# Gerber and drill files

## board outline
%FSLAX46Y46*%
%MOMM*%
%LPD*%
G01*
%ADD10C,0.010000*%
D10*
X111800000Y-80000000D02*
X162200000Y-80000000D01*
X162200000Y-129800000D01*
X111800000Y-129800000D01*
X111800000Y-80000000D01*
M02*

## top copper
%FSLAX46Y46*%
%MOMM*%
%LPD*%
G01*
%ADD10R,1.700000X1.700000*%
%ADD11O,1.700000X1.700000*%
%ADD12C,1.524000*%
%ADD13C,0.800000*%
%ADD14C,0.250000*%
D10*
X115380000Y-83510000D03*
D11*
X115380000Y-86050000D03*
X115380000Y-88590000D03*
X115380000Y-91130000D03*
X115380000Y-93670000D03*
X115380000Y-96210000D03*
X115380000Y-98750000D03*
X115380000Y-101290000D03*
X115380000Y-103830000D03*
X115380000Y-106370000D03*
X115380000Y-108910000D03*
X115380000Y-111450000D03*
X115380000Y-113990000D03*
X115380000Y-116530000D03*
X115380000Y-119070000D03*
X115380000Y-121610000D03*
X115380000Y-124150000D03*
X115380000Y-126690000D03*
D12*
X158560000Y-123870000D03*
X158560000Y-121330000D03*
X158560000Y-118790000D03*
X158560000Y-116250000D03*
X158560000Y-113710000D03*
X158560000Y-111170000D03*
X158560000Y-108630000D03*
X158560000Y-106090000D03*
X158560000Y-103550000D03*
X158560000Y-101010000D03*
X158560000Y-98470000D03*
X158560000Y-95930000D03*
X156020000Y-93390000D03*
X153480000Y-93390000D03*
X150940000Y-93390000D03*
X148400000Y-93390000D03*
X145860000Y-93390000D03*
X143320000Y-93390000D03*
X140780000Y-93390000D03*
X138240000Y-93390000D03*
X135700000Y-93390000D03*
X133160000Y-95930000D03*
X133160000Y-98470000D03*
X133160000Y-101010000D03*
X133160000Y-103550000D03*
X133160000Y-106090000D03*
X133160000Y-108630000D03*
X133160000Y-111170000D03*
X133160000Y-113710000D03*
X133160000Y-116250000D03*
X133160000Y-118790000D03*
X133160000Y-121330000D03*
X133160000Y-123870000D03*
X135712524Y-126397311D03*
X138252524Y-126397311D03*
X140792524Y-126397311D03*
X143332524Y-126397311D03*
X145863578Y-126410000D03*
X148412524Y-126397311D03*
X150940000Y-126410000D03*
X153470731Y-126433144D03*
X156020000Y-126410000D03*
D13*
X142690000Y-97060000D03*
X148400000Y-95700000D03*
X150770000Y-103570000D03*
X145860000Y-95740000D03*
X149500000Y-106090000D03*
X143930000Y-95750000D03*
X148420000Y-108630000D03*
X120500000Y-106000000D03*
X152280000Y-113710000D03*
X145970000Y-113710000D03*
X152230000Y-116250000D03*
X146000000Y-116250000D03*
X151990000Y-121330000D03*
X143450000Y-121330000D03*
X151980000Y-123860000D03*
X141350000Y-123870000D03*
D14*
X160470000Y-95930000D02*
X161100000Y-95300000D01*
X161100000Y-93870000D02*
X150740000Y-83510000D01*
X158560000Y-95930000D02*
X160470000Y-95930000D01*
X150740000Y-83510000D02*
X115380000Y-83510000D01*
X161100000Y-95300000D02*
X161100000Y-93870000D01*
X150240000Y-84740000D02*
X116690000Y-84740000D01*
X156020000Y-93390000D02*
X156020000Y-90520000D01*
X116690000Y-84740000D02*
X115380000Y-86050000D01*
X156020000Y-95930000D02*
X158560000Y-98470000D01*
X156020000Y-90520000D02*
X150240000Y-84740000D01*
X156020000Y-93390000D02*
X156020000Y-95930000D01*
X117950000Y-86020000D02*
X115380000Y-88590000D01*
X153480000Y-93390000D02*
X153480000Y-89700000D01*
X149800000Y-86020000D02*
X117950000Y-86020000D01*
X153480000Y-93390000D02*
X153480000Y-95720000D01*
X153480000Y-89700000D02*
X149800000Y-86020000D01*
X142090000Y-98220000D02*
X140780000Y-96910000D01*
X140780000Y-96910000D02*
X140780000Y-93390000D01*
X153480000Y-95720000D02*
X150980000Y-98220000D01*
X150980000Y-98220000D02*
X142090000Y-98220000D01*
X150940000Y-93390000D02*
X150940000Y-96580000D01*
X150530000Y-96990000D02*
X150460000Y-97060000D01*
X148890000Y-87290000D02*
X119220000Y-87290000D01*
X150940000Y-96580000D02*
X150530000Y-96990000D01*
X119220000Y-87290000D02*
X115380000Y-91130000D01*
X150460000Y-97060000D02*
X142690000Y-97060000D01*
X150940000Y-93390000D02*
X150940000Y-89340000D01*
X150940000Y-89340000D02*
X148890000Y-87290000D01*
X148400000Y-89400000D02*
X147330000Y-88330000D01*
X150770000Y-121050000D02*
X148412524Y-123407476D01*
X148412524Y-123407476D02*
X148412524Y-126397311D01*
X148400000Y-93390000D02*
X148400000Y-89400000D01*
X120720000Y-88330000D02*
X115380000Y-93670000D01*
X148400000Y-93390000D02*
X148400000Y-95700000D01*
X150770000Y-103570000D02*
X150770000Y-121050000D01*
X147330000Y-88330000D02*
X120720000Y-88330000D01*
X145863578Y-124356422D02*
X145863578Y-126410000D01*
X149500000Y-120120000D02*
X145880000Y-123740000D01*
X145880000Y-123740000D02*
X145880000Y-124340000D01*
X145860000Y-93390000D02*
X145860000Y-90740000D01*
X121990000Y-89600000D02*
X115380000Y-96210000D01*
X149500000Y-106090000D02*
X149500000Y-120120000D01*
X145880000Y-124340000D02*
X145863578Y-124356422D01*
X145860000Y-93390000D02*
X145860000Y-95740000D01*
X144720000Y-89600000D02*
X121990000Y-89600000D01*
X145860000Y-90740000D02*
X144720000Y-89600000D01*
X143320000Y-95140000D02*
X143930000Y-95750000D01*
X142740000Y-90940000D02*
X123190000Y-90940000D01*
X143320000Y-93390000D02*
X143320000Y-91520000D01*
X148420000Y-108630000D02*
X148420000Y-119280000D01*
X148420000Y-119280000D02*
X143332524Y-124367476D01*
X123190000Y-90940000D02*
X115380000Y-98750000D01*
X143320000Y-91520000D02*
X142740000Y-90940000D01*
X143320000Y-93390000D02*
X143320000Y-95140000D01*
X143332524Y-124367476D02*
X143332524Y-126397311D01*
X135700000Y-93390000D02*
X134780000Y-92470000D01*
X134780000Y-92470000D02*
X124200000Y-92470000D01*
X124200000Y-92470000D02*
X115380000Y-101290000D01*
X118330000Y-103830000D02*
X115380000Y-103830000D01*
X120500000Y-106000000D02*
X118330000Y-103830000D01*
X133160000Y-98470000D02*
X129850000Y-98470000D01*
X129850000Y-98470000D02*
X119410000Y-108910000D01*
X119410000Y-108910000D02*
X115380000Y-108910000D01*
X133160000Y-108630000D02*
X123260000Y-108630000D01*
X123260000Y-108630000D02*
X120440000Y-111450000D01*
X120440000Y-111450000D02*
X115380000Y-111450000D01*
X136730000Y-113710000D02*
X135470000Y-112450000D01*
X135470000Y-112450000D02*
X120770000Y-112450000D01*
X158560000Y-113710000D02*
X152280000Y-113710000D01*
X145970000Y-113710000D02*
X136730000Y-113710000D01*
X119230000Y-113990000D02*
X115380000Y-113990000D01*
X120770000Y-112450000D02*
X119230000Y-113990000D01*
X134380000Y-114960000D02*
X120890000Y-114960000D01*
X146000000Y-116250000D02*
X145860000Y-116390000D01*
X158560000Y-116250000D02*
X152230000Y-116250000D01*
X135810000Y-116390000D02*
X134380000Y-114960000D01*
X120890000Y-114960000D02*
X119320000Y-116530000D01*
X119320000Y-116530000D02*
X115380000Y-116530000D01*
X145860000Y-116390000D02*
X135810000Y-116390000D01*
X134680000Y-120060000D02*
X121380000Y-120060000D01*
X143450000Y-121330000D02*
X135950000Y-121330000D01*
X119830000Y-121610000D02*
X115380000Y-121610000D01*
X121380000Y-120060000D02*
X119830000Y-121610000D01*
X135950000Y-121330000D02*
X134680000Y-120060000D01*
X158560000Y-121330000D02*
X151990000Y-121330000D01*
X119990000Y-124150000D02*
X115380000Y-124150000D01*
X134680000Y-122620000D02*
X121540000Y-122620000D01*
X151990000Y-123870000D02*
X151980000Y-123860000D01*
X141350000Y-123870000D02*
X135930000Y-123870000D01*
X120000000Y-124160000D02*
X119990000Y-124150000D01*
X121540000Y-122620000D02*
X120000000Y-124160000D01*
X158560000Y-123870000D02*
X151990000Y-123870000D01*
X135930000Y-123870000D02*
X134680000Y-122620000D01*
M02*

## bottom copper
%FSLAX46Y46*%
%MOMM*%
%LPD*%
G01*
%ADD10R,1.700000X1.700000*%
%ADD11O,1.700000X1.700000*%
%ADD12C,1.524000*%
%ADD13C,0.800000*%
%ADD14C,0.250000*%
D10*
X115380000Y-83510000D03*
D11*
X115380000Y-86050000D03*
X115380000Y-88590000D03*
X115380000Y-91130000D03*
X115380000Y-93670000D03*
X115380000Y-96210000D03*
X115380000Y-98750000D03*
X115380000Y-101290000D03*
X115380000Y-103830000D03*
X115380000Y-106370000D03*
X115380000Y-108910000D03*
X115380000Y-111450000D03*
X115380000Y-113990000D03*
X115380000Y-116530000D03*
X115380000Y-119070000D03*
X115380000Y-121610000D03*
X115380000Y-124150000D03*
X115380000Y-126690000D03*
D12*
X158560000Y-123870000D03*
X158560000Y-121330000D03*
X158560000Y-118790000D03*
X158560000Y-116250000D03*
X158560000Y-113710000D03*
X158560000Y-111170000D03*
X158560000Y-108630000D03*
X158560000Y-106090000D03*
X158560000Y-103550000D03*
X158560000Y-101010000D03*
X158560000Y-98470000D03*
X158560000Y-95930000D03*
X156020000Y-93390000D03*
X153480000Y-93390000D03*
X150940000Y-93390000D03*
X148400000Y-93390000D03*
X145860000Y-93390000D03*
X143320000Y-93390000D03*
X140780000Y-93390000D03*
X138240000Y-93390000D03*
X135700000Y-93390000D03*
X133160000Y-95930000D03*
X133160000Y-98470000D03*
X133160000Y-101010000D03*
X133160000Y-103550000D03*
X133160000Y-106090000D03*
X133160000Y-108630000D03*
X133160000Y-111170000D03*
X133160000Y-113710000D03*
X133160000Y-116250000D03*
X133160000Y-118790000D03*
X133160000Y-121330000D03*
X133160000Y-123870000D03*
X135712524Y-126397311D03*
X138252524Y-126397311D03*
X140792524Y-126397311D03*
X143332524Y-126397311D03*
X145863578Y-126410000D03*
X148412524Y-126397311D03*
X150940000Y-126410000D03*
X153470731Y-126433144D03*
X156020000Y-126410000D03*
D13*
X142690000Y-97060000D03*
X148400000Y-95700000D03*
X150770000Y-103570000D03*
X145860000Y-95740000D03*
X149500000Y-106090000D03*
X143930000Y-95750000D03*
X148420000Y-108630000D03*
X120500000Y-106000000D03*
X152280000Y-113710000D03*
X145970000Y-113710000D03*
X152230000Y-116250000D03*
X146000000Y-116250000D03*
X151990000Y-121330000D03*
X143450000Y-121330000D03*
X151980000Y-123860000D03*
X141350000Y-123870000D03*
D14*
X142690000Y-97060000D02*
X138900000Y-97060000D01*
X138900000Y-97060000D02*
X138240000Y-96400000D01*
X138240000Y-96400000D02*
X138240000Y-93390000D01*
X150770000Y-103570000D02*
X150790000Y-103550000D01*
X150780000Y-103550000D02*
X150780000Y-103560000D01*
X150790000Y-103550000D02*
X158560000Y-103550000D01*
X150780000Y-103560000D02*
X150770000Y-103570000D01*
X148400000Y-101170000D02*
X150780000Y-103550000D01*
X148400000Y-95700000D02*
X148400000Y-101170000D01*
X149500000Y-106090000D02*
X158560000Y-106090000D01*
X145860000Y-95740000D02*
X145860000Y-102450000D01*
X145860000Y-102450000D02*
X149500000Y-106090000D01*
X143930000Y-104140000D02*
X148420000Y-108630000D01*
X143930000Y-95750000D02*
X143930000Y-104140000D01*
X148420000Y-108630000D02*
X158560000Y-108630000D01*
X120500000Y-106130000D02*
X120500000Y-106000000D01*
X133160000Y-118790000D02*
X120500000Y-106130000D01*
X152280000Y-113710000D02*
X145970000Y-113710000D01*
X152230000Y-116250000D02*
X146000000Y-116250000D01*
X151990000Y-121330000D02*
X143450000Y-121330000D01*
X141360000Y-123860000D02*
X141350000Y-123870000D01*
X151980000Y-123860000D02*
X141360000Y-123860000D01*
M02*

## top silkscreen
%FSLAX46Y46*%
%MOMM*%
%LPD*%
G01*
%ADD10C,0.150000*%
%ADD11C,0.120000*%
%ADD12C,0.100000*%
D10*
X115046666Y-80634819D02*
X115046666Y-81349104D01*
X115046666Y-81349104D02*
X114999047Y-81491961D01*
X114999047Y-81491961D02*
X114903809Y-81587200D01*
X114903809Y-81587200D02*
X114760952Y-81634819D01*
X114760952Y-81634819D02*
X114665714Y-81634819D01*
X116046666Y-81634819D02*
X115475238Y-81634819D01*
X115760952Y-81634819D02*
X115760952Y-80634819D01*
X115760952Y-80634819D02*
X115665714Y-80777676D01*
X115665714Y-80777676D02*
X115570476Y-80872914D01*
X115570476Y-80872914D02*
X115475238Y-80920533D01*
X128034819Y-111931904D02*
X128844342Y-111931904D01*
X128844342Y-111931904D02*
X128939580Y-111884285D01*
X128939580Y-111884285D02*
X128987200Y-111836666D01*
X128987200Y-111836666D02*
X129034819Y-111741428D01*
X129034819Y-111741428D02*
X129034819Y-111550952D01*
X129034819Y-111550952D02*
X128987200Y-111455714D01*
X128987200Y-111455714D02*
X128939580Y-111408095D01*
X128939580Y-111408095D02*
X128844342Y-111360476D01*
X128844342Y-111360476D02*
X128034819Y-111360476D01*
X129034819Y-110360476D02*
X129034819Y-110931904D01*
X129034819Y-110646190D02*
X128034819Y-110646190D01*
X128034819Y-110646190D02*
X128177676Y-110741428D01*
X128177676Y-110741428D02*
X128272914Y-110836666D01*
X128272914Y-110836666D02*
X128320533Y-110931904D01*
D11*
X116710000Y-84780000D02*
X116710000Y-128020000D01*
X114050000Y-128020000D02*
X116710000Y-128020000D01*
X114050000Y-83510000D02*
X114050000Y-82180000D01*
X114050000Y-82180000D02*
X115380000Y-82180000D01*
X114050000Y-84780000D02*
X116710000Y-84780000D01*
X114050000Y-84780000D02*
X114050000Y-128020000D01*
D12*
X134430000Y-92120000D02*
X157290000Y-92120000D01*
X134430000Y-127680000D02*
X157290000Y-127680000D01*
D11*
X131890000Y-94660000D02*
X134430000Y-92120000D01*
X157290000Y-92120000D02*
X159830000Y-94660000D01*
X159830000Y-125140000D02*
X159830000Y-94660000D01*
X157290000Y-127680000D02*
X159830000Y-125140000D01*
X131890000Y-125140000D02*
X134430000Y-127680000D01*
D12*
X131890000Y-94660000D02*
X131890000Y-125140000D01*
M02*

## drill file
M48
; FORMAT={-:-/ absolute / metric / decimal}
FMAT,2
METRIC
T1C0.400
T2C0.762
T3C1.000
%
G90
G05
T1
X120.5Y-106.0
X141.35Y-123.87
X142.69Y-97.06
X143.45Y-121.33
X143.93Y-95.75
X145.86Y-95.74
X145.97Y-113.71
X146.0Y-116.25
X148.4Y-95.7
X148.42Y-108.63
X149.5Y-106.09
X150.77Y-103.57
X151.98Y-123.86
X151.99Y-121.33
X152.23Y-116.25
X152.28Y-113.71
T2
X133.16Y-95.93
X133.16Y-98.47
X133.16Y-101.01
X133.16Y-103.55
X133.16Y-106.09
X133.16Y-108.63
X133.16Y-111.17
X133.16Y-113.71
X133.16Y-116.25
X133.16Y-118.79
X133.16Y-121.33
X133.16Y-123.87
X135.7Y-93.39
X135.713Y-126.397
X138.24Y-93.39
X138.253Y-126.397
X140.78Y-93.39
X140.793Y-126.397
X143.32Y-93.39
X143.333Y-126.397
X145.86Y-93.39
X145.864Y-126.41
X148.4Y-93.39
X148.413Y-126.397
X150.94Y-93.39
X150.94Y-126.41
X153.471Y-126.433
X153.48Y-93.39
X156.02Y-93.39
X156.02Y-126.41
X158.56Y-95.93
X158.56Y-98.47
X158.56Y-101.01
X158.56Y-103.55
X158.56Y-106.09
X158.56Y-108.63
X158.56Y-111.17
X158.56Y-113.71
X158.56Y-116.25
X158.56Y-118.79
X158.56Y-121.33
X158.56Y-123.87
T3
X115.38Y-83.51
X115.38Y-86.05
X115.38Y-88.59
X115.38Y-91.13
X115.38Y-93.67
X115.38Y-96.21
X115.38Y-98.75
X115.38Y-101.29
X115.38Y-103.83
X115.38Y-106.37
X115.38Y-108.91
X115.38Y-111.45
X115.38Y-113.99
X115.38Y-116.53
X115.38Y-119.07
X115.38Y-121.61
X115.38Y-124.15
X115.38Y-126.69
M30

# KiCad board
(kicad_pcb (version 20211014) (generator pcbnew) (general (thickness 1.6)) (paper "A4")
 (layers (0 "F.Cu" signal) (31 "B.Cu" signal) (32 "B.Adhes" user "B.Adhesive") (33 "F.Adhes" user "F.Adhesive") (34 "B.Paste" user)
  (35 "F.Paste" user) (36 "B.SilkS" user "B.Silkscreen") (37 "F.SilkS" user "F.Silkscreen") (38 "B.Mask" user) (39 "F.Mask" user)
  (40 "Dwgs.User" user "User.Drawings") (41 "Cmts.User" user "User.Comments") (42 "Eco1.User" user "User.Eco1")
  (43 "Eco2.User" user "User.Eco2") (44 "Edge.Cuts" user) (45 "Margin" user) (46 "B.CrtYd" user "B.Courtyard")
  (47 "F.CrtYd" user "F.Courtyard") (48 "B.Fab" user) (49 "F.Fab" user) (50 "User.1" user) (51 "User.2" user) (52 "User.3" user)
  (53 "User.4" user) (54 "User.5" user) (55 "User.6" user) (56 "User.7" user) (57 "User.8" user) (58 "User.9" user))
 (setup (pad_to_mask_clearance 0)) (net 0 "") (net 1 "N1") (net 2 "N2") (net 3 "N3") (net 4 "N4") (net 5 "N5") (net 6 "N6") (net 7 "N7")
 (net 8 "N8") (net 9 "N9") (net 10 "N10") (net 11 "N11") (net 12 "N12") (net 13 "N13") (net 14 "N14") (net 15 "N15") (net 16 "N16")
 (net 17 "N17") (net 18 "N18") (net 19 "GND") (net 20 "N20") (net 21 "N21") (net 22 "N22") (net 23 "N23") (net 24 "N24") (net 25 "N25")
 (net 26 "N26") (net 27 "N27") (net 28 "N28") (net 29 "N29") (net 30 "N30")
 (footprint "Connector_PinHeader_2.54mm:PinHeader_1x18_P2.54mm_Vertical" (layer "F.Cu") (at 115.38 83.51)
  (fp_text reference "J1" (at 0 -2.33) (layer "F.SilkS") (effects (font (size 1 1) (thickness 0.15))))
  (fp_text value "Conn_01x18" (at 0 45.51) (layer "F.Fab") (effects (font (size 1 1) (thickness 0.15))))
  (fp_line (start 1.33 1.27) (end 1.33 44.51) (layer "F.SilkS") (width 0.12))
  (fp_line (start -1.33 44.51) (end 1.33 44.51) (layer "F.SilkS") (width 0.12))
  (fp_line (start -1.33 0) (end -1.33 -1.33) (layer "F.SilkS") (width 0.12))
  (fp_line (start -1.33 -1.33) (end 0 -1.33) (layer "F.SilkS") (width 0.12))
  (fp_line (start -1.33 1.27) (end 1.33 1.27) (layer "F.SilkS") (width 0.12))
  (fp_line (start -1.33 1.27) (end -1.33 44.51) (layer "F.SilkS") (width 0.12))
  (pad "1" thru_hole rect locked (at 0 0) (size 1.7 1.7) (drill 1) (layers *.Cu *.Mask) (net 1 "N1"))
  (pad "2" thru_hole oval locked (at 0 2.54) (size 1.7 1.7) (drill 1) (layers *.Cu *.Mask) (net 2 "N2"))
  (pad "3" thru_hole oval locked (at 0 5.08) (size 1.7 1.7) (drill 1) (layers *.Cu *.Mask) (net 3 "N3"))
  (pad "4" thru_hole oval locked (at 0 7.62) (size 1.7 1.7) (drill 1) (layers *.Cu *.Mask) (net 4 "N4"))
  (pad "5" thru_hole oval locked (at 0 10.16) (size 1.7 1.7) (drill 1) (layers *.Cu *.Mask) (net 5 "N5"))
  (pad "6" thru_hole oval locked (at 0 12.7) (size 1.7 1.7) (drill 1) (layers *.Cu *.Mask) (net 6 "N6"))
  (pad "7" thru_hole oval locked (at 0 15.24) (size 1.7 1.7) (drill 1) (layers *.Cu *.Mask) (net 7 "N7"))
  (pad "8" thru_hole oval locked (at 0 17.78) (size 1.7 1.7) (drill 1) (layers *.Cu *.Mask) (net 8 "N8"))
  (pad "9" thru_hole oval locked (at 0 20.32) (size 1.7 1.7) (drill 1) (layers *.Cu *.Mask) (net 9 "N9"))
  (pad "10" thru_hole oval locked (at 0 22.86) (size 1.7 1.7) (drill 1) (layers *.Cu *.Mask) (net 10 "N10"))
  (pad "11" thru_hole oval locked (at 0 25.4) (size 1.7 1.7) (drill 1) (layers *.Cu *.Mask) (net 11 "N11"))
  (pad "12" thru_hole oval locked (at 0 27.94) (size 1.7 1.7) (drill 1) (layers *.Cu *.Mask) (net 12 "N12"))
  (pad "13" thru_hole oval locked (at 0 30.48) (size 1.7 1.7) (drill 1) (layers *.Cu *.Mask) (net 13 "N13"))
  (pad "14" thru_hole oval locked (at 0 33.02) (size 1.7 1.7) (drill 1) (layers *.Cu *.Mask) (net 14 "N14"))
  (pad "15" thru_hole oval locked (at 0 35.56) (size 1.7 1.7) (drill 1) (layers *.Cu *.Mask) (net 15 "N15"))
  (pad "16" thru_hole oval locked (at 0 38.1) (size 1.7 1.7) (drill 1) (layers *.Cu *.Mask) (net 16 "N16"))
  (pad "17" thru_hole oval locked (at 0 40.64) (size 1.7 1.7) (drill 1) (layers *.Cu *.Mask) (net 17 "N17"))
  (pad "18" thru_hole oval locked (at 0 43.18) (size 1.7 1.7) (drill 1) (layers *.Cu *.Mask) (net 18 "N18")))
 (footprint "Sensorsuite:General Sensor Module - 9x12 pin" (layer "F.Cu") (at 145.86 111.17 90)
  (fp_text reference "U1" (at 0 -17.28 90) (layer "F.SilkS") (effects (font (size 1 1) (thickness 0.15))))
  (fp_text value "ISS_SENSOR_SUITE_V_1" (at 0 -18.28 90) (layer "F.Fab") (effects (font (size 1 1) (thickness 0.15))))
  (fp_line (start 19.05 -11.43) (end 19.05 11.43) (layer "F.SilkS") (width 0.1))
  (fp_line (start -16.51 -11.43) (end -16.51 11.43) (layer "F.SilkS") (width 0.1))
  (fp_line (start 16.51 -13.97) (end 19.05 -11.43) (layer "F.SilkS") (width 0.12))
  (fp_line (start 19.05 11.43) (end 16.51 13.97) (layer "F.SilkS") (width 0.12))
  (fp_line (start -13.97 13.97) (end 16.51 13.97) (layer "F.SilkS") (width 0.12))
  (fp_line (start -16.51 11.43) (end -13.97 13.97) (layer "F.SilkS") (width 0.12))
  (fp_line (start -13.97 -13.97) (end -16.51 -11.43) (layer "F.SilkS") (width 0.12))
  (fp_line (start 16.51 -13.97) (end -13.97 -13.97) (layer "F.SilkS") (width 0.1))
  (pad "1" thru_hole circle (at -12.7 12.7 90) (size 1.524 1.524) (drill 0.762) (layers *.Cu *.Mask) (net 17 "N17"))
  (pad "2" thru_hole circle (at -10.16 12.7 90) (size 1.524 1.524) (drill 0.762) (layers *.Cu *.Mask) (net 16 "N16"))
  (pad "3" thru_hole circle (at -7.62 12.7 90) (size 1.524 1.524) (drill 0.762) (layers *.Cu *.Mask) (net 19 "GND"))
  (pad "4" thru_hole circle (at -5.08 12.7 90) (size 1.524 1.524) (drill 0.762) (layers *.Cu *.Mask) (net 14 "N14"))
  (pad "5" thru_hole circle (at -2.54 12.7 90) (size 1.524 1.524) (drill 0.762) (layers *.Cu *.Mask) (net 13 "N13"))
  (pad "6" thru_hole circle (at 0 12.7 90) (size 1.524 1.524) (drill 0.762) (layers *.Cu *.Mask) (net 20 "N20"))
  (pad "7" thru_hole circle (at 2.54 12.7 90) (size 1.524 1.524) (drill 0.762) (layers *.Cu *.Mask) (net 7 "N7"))
  (pad "8" thru_hole circle (at 5.08 12.7 90) (size 1.524 1.524) (drill 0.762) (layers *.Cu *.Mask) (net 6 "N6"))
  (pad "9" thru_hole circle (at 7.62 12.7 90) (size 1.524 1.524) (drill 0.762) (layers *.Cu *.Mask) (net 5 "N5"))
  (pad "10" thru_hole circle (at 10.16 12.7 90) (size 1.524 1.524) (drill 0.762) (layers *.Cu *.Mask) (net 1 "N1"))
  (pad "11" thru_hole circle (at 12.7 12.7 90) (size 1.524 1.524) (drill 0.762) (layers *.Cu *.Mask) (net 2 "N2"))
  (pad "12" thru_hole circle (at 15.24 12.7 90) (size 1.524 1.524) (drill 0.762) (layers *.Cu *.Mask) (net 1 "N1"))
  (pad "13" thru_hole circle (at 17.78 10.16 90) (size 1.524 1.524) (drill 0.762) (layers *.Cu *.Mask) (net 2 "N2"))
  (pad "14" thru_hole circle (at 17.78 7.62 90) (size 1.524 1.524) (drill 0.762) (layers *.Cu *.Mask) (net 3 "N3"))
  (pad "15" thru_hole circle (at 17.78 5.08 90) (size 1.524 1.524) (drill 0.762) (layers *.Cu *.Mask) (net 4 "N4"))
  (pad "16" thru_hole circle (at 17.78 2.54 90) (size 1.524 1.524) (drill 0.762) (layers *.Cu *.Mask) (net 5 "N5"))
  (pad "17" thru_hole circle (at 17.78 0 90) (size 1.524 1.524) (drill 0.762) (layers *.Cu *.Mask) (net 6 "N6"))
  (pad "18" thru_hole circle (at 17.78 -2.54 90) (size 1.524 1.524) (drill 0.762) (layers *.Cu *.Mask) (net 7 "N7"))
  (pad "19" thru_hole circle (at 17.78 -5.08 90) (size 1.524 1.524) (drill 0.762) (layers *.Cu *.Mask) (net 3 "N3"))
  (pad "20" thru_hole circle (at 17.78 -7.62 90) (size 1.524 1.524) (drill 0.762) (layers *.Cu *.Mask) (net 4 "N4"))
  (pad "21" thru_hole circle (at 17.78 -10.16 90) (size 1.524 1.524) (drill 0.762) (layers *.Cu *.Mask) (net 8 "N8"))
  (pad "22" thru_hole circle (at 15.24 -12.7 90) (size 1.524 1.524) (drill 0.762) (layers *.Cu *.Mask) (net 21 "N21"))
  (pad "23" thru_hole circle (at 12.7 -12.7 90) (size 1.524 1.524) (drill 0.762) (layers *.Cu *.Mask) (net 11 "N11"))
  (pad "24" thru_hole circle (at 10.16 -12.7 90) (size 1.524 1.524) (drill 0.762) (layers *.Cu *.Mask) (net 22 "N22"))
  (pad "25" thru_hole circle (at 7.62 -12.7 90) (size 1.524 1.524) (drill 0.762) (layers *.Cu *.Mask))
  (pad "26" thru_hole circle (at 5.08 -12.7 90) (size 1.524 1.524) (drill 0.762) (layers *.Cu *.Mask) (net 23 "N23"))
  (pad "27" thru_hole circle (at 2.54 -12.7 90) (size 1.524 1.524) (drill 0.762) (layers *.Cu *.Mask) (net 12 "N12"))
  (pad "28" thru_hole circle (at 0 -12.7 90) (size 1.524 1.524) (drill 0.762) (layers *.Cu *.Mask) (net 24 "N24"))
  (pad "29" thru_hole circle (at -2.54 -12.7 90) (size 1.524 1.524) (drill 0.762) (layers *.Cu *.Mask) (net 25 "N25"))
  (pad "30" thru_hole circle (at -5.08 -12.7 90) (size 1.524 1.524) (drill 0.762) (layers *.Cu *.Mask))
  (pad "31" thru_hole circle (at -7.62 -12.7 90) (size 1.524 1.524) (drill 0.762) (layers *.Cu *.Mask) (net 9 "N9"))
  (pad "32" thru_hole circle (at -10.16 -12.7 90) (size 1.524 1.524) (drill 0.762) (layers *.Cu *.Mask) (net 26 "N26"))
  (pad "33" thru_hole circle (at -12.7 -12.7 90) (size 1.524 1.524) (drill 0.762) (layers *.Cu *.Mask))
  (pad "34" thru_hole circle (at -15.227311 -10.147476 90) (size 1.524 1.524) (drill 0.762) (layers *.Cu *.Mask))
  (pad "35" thru_hole circle (at -15.227311 -7.607476 90) (size 1.524 1.524) (drill 0.762) (layers *.Cu *.Mask))
  (pad "36" thru_hole circle (at -15.227311 -5.067476 90) (size 1.524 1.524) (drill 0.762) (layers *.Cu *.Mask) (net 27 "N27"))
  (pad "37" thru_hole circle (at -15.227311 -2.527476 90) (size 1.524 1.524) (drill 0.762) (layers *.Cu *.Mask) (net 7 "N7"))
  (pad "38" thru_hole circle (at -15.24 0.003578 90) (size 1.524 1.524) (drill 0.762) (layers *.Cu *.Mask) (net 6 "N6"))
  (pad "39" thru_hole circle (at -15.227311 2.552524 90) (size 1.524 1.524) (drill 0.762) (layers *.Cu *.Mask) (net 5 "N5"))
  (pad "40" thru_hole circle (at -15.24 5.08 90) (size 1.524 1.524) (drill 0.762) (layers *.Cu *.Mask) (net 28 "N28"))
  (pad "41" thru_hole circle (at -15.263144 7.610731 90) (size 1.524 1.524) (drill 0.762) (layers *.Cu *.Mask) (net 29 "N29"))
  (pad "42" thru_hole circle (at -15.24 10.16 90) (size 1.524 1.524) (drill 0.762) (layers *.Cu *.Mask) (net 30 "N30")))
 (gr_rect (start 111.8 80) (end 162.2 129.8) (layer "Edge.Cuts") (width 0.01) (fill none))
 (segment (start 160.47 95.93) (end 161.1 95.3) (width 0.25) (layer "F.Cu") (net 1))
 (segment (start 161.1 93.87) (end 150.74 83.51) (width 0.25) (layer "F.Cu") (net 1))
 (segment (start 158.56 95.93) (end 160.47 95.93) (width 0.25) (layer "F.Cu") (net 1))
 (segment (start 150.74 83.51) (end 115.38 83.51) (width 0.25) (layer "F.Cu") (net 1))
 (segment (start 161.1 95.3) (end 161.1 93.87) (width 0.25) (layer "F.Cu") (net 1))
 (segment (start 150.24 84.74) (end 116.69 84.74) (width 0.25) (layer "F.Cu") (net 2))
 (segment (start 156.02 93.39) (end 156.02 90.52) (width 0.25) (layer "F.Cu") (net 2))
 (segment (start 116.69 84.74) (end 115.38 86.05) (width 0.25) (layer "F.Cu") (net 2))
 (segment (start 156.02 95.93) (end 158.56 98.47) (width 0.25) (layer "F.Cu") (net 2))
 (segment (start 156.02 90.52) (end 150.24 84.74) (width 0.25) (layer "F.Cu") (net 2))
 (segment (start 156.02 93.39) (end 156.02 95.93) (width 0.25) (layer "F.Cu") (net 2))
 (segment (start 117.95 86.02) (end 115.38 88.59) (width 0.25) (layer "F.Cu") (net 3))
 (segment (start 153.48 93.39) (end 153.48 89.7) (width 0.25) (layer "F.Cu") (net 3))
 (segment (start 149.8 86.02) (end 117.95 86.02) (width 0.25) (layer "F.Cu") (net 3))
 (segment (start 153.48 93.39) (end 153.48 95.72) (width 0.25) (layer "F.Cu") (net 3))
 (segment (start 153.48 89.7) (end 149.8 86.02) (width 0.25) (layer "F.Cu") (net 3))
 (segment (start 142.09 98.22) (end 140.78 96.91) (width 0.25) (layer "F.Cu") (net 3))
 (segment (start 140.78 96.91) (end 140.78 93.39) (width 0.25) (layer "F.Cu") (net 3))
 (segment (start 153.48 95.72) (end 150.98 98.22) (width 0.25) (layer "F.Cu") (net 3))
 (segment (start 150.98 98.22) (end 142.09 98.22) (width 0.25) (layer "F.Cu") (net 3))
 (segment (start 150.94 93.39) (end 150.94 96.58) (width 0.25) (layer "F.Cu") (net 4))
 (segment (start 150.53 96.99) (end 150.46 97.06) (width 0.25) (layer "F.Cu") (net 4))
 (segment (start 148.89 87.29) (end 119.22 87.29) (width 0.25) (layer "F.Cu") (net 4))
 (segment (start 150.94 96.58) (end 150.53 96.99) (width 0.25) (layer "F.Cu") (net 4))
 (segment (start 119.22 87.29) (end 115.38 91.13) (width 0.25) (layer "F.Cu") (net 4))
 (segment (start 150.46 97.06) (end 142.69 97.06) (width 0.25) (layer "F.Cu") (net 4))
 (segment (start 150.94 93.39) (end 150.94 89.34) (width 0.25) (layer "F.Cu") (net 4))
 (segment (start 150.94 89.34) (end 148.89 87.29) (width 0.25) (layer "F.Cu") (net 4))
 (via (at 142.69 97.06) (size 0.8) (drill 0.4) (layers "F.Cu" "B.Cu") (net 4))
 (segment (start 142.69 97.06) (end 138.9 97.06) (width 0.25) (layer "B.Cu") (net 4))
 (segment (start 138.9 97.06) (end 138.24 96.4) (width 0.25) (layer "B.Cu") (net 4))
 (segment (start 138.24 96.4) (end 138.24 93.39) (width 0.25) (layer "B.Cu") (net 4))
 (segment (start 148.4 89.4) (end 147.33 88.33) (width 0.25) (layer "F.Cu") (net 5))
 (segment (start 150.77 121.05) (end 148.412524 123.407476) (width 0.25) (layer "F.Cu") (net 5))
 (segment (start 148.412524 123.407476) (end 148.412524 126.397311) (width 0.25) (layer "F.Cu") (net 5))
 (segment (start 148.4 93.39) (end 148.4 89.4) (width 0.25) (layer "F.Cu") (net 5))
 (segment (start 120.72 88.33) (end 115.38 93.67) (width 0.25) (layer "F.Cu") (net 5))
 (segment (start 148.4 93.39) (end 148.4 95.7) (width 0.25) (layer "F.Cu") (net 5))
 (segment (start 150.77 103.57) (end 150.77 121.05) (width 0.25) (layer "F.Cu") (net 5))
 (segment (start 147.33 88.33) (end 120.72 88.33) (width 0.25) (layer "F.Cu") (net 5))
 (via (at 148.4 95.7) (size 0.8) (drill 0.4) (layers "F.Cu" "B.Cu") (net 5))
 (via (at 150.77 103.57) (size 0.8) (drill 0.4) (layers "F.Cu" "B.Cu") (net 5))
 (segment (start 150.77 103.57) (end 150.79 103.55) (width 0.25) (layer "B.Cu") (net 5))
 (segment (start 150.78 103.55) (end 150.78 103.56) (width 0.25) (layer "B.Cu") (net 5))
 (segment (start 150.79 103.55) (end 158.56 103.55) (width 0.25) (layer "B.Cu") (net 5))
 (segment (start 150.78 103.56) (end 150.77 103.57) (width 0.25) (layer "B.Cu") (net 5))
 (segment (start 148.4 101.17) (end 150.78 103.55) (width 0.25) (layer "B.Cu") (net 5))
 (segment (start 148.4 95.7) (end 148.4 101.17) (width 0.25) (layer "B.Cu") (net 5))
 (segment (start 145.863578 124.356422) (end 145.863578 126.41) (width 0.25) (layer "F.Cu") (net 6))
 (segment (start 149.5 120.12) (end 145.88 123.74) (width 0.25) (layer "F.Cu") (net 6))
 (segment (start 145.88 123.74) (end 145.88 124.34) (width 0.25) (layer "F.Cu") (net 6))
 (segment (start 145.86 93.39) (end 145.86 90.74) (width 0.25) (layer "F.Cu") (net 6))
 (segment (start 121.99 89.6) (end 115.38 96.21) (width 0.25) (layer "F.Cu") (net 6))
 (segment (start 149.5 106.09) (end 149.5 120.12) (width 0.25) (layer "F.Cu") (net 6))
 (segment (start 145.88 124.34) (end 145.863578 124.356422) (width 0.25) (layer "F.Cu") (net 6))
 (segment (start 145.86 93.39) (end 145.86 95.74) (width 0.25) (layer "F.Cu") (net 6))
 (segment (start 144.72 89.6) (end 121.99 89.6) (width 0.25) (layer "F.Cu") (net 6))
 (segment (start 145.86 90.74) (end 144.72 89.6) (width 0.25) (layer "F.Cu") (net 6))
 (via (at 145.86 95.74) (size 0.8) (drill 0.4) (layers "F.Cu" "B.Cu") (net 6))
 (via (at 149.5 106.09) (size 0.8) (drill 0.4) (layers "F.Cu" "B.Cu") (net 6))
 (segment (start 149.5 106.09) (end 158.56 106.09) (width 0.25) (layer "B.Cu") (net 6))
 (segment (start 145.86 95.74) (end 145.86 102.45) (width 0.25) (layer "B.Cu") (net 6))
 (segment (start 145.86 102.45) (end 149.5 106.09) (width 0.25) (layer "B.Cu") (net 6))
 (segment (start 143.32 95.14) (end 143.93 95.75) (width 0.25) (layer "F.Cu") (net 7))
 (segment (start 142.74 90.94) (end 123.19 90.94) (width 0.25) (layer "F.Cu") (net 7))
 (segment (start 143.32 93.39) (end 143.32 91.52) (width 0.25) (layer "F.Cu") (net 7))
 (segment (start 148.42 108.63) (end 148.42 119.28) (width 0.25) (layer "F.Cu") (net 7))
 (segment (start 148.42 119.28) (end 143.332524 124.367476) (width 0.25) (layer "F.Cu") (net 7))
 (segment (start 123.19 90.94) (end 115.38 98.75) (width 0.25) (layer "F.Cu") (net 7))
 (segment (start 143.32 91.52) (end 142.74 90.94) (width 0.25) (layer "F.Cu") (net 7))
 (segment (start 143.32 93.39) (end 143.32 95.14) (width 0.25) (layer "F.Cu") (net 7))
 (segment (start 143.332524 124.367476) (end 143.332524 126.397311) (width 0.25) (layer "F.Cu") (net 7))
 (via (at 143.93 95.75) (size 0.8) (drill 0.4) (layers "F.Cu" "B.Cu") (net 7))
 (via (at 148.42 108.63) (size 0.8) (drill 0.4) (layers "F.Cu" "B.Cu") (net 7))
 (segment (start 143.93 104.14) (end 148.42 108.63) (width 0.25) (layer "B.Cu") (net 7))
 (segment (start 143.93 95.75) (end 143.93 104.14) (width 0.25) (layer "B.Cu") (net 7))
 (segment (start 148.42 108.63) (end 158.56 108.63) (width 0.25) (layer "B.Cu") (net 7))
 (segment (start 135.7 93.39) (end 134.78 92.47) (width 0.25) (layer "F.Cu") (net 8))
 (segment (start 134.78 92.47) (end 124.2 92.47) (width 0.25) (layer "F.Cu") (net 8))
 (segment (start 124.2 92.47) (end 115.38 101.29) (width 0.25) (layer "F.Cu") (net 8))
 (segment (start 118.33 103.83) (end 115.38 103.83) (width 0.25) (layer "F.Cu") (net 9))
 (segment (start 120.5 106) (end 118.33 103.83) (width 0.25) (layer "F.Cu") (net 9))
 (via (at 120.5 106) (size 0.8) (drill 0.4) (layers "F.Cu" "B.Cu") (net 9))
 (segment (start 120.5 106.13) (end 120.5 106) (width 0.25) (layer "B.Cu") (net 9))
 (segment (start 133.16 118.79) (end 120.5 106.13) (width 0.25) (layer "B.Cu") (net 9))
 (segment (start 133.16 98.47) (end 129.85 98.47) (width 0.25) (layer "F.Cu") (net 11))
 (segment (start 129.85 98.47) (end 119.41 108.91) (width 0.25) (layer "F.Cu") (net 11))
 (segment (start 119.41 108.91) (end 115.38 108.91) (width 0.25) (layer "F.Cu") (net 11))
 (segment (start 133.16 108.63) (end 123.26 108.63) (width 0.25) (layer "F.Cu") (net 12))
 (segment (start 123.26 108.63) (end 120.44 111.45) (width 0.25) (layer "F.Cu") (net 12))
 (segment (start 120.44 111.45) (end 115.38 111.45) (width 0.25) (layer "F.Cu") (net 12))
 (segment (start 136.73 113.71) (end 135.47 112.45) (width 0.25) (layer "F.Cu") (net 13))
 (segment (start 135.47 112.45) (end 120.77 112.45) (width 0.25) (layer "F.Cu") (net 13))
 (segment (start 158.56 113.71) (end 152.28 113.71) (width 0.25) (layer "F.Cu") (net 13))
 (segment (start 145.97 113.71) (end 136.73 113.71) (width 0.25) (layer "F.Cu") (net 13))
 (segment (start 119.23 113.99) (end 115.38 113.99) (width 0.25) (layer "F.Cu") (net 13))
 (segment (start 120.77 112.45) (end 119.23 113.99) (width 0.25) (layer "F.Cu") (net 13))
 (via (at 152.28 113.71) (size 0.8) (drill 0.4) (layers "F.Cu" "B.Cu") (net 13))
 (via (at 145.97 113.71) (size 0.8) (drill 0.4) (layers "F.Cu" "B.Cu") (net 13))
 (segment (start 152.28 113.71) (end 145.97 113.71) (width 0.25) (layer "B.Cu") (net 13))
 (segment (start 134.38 114.96) (end 120.89 114.96) (width 0.25) (layer "F.Cu") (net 14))
 (segment (start 146 116.25) (end 145.86 116.39) (width 0.25) (layer "F.Cu") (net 14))
 (segment (start 158.56 116.25) (end 152.23 116.25) (width 0.25) (layer "F.Cu") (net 14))
 (segment (start 135.81 116.39) (end 134.38 114.96) (width 0.25) (layer "F.Cu") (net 14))
 (segment (start 120.89 114.96) (end 119.32 116.53) (width 0.25) (layer "F.Cu") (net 14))
 (segment (start 119.32 116.53) (end 115.38 116.53) (width 0.25) (layer "F.Cu") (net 14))
 (segment (start 145.86 116.39) (end 135.81 116.39) (width 0.25) (layer "F.Cu") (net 14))
 (via (at 152.23 116.25) (size 0.8) (drill 0.4) (layers "F.Cu" "B.Cu") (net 14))
 (via (at 146 116.25) (size 0.8) (drill 0.4) (layers "F.Cu" "B.Cu") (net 14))
 (segment (start 152.23 116.25) (end 146 116.25) (width 0.25) (layer "B.Cu") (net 14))
 (segment (start 134.68 120.06) (end 121.38 120.06) (width 0.25) (layer "F.Cu") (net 16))
 (segment (start 143.45 121.33) (end 135.95 121.33) (width 0.25) (layer "F.Cu") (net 16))
 (segment (start 119.83 121.61) (end 115.38 121.61) (width 0.25) (layer "F.Cu") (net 16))
 (segment (start 121.38 120.06) (end 119.83 121.61) (width 0.25) (layer "F.Cu") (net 16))
 (segment (start 135.95 121.33) (end 134.68 120.06) (width 0.25) (layer "F.Cu") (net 16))
 (segment (start 158.56 121.33) (end 151.99 121.33) (width 0.25) (layer "F.Cu") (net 16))
 (via (at 151.99 121.33) (size 0.8) (drill 0.4) (layers "F.Cu" "B.Cu") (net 16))
 (via (at 143.45 121.33) (size 0.8) (drill 0.4) (layers "F.Cu" "B.Cu") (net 16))
 (segment (start 151.99 121.33) (end 143.45 121.33) (width 0.25) (layer "B.Cu") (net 16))
 (segment (start 119.99 124.15) (end 115.38 124.15) (width 0.25) (layer "F.Cu") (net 17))
 (segment (start 134.68 122.62) (end 121.54 122.62) (width 0.25) (layer "F.Cu") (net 17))
 (segment (start 151.99 123.87) (end 151.98 123.86) (width 0.25) (layer "F.Cu") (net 17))
 (segment (start 141.35 123.87) (end 135.93 123.87) (width 0.25) (layer "F.Cu") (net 17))
 (segment (start 120 124.16) (end 119.99 124.15) (width 0.25) (layer "F.Cu") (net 17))
 (segment (start 121.54 122.62) (end 120 124.16) (width 0.25) (layer "F.Cu") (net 17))
 (segment (start 158.56 123.87) (end 151.99 123.87) (width 0.25) (layer "F.Cu") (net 17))
 (segment (start 135.93 123.87) (end 134.68 122.62) (width 0.25) (layer "F.Cu") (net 17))
 (via (at 151.98 123.86) (size 0.8) (drill 0.4) (layers "F.Cu" "B.Cu") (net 17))
 (via (at 141.35 123.87) (size 0.8) (drill 0.4) (layers "F.Cu" "B.Cu") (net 17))
 (segment (start 141.36 123.86) (end 141.35 123.87) (width 0.25) (layer "B.Cu") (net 17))
 (segment (start 151.98 123.86) (end 141.36 123.86) (width 0.25) (layer "B.Cu") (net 17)))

